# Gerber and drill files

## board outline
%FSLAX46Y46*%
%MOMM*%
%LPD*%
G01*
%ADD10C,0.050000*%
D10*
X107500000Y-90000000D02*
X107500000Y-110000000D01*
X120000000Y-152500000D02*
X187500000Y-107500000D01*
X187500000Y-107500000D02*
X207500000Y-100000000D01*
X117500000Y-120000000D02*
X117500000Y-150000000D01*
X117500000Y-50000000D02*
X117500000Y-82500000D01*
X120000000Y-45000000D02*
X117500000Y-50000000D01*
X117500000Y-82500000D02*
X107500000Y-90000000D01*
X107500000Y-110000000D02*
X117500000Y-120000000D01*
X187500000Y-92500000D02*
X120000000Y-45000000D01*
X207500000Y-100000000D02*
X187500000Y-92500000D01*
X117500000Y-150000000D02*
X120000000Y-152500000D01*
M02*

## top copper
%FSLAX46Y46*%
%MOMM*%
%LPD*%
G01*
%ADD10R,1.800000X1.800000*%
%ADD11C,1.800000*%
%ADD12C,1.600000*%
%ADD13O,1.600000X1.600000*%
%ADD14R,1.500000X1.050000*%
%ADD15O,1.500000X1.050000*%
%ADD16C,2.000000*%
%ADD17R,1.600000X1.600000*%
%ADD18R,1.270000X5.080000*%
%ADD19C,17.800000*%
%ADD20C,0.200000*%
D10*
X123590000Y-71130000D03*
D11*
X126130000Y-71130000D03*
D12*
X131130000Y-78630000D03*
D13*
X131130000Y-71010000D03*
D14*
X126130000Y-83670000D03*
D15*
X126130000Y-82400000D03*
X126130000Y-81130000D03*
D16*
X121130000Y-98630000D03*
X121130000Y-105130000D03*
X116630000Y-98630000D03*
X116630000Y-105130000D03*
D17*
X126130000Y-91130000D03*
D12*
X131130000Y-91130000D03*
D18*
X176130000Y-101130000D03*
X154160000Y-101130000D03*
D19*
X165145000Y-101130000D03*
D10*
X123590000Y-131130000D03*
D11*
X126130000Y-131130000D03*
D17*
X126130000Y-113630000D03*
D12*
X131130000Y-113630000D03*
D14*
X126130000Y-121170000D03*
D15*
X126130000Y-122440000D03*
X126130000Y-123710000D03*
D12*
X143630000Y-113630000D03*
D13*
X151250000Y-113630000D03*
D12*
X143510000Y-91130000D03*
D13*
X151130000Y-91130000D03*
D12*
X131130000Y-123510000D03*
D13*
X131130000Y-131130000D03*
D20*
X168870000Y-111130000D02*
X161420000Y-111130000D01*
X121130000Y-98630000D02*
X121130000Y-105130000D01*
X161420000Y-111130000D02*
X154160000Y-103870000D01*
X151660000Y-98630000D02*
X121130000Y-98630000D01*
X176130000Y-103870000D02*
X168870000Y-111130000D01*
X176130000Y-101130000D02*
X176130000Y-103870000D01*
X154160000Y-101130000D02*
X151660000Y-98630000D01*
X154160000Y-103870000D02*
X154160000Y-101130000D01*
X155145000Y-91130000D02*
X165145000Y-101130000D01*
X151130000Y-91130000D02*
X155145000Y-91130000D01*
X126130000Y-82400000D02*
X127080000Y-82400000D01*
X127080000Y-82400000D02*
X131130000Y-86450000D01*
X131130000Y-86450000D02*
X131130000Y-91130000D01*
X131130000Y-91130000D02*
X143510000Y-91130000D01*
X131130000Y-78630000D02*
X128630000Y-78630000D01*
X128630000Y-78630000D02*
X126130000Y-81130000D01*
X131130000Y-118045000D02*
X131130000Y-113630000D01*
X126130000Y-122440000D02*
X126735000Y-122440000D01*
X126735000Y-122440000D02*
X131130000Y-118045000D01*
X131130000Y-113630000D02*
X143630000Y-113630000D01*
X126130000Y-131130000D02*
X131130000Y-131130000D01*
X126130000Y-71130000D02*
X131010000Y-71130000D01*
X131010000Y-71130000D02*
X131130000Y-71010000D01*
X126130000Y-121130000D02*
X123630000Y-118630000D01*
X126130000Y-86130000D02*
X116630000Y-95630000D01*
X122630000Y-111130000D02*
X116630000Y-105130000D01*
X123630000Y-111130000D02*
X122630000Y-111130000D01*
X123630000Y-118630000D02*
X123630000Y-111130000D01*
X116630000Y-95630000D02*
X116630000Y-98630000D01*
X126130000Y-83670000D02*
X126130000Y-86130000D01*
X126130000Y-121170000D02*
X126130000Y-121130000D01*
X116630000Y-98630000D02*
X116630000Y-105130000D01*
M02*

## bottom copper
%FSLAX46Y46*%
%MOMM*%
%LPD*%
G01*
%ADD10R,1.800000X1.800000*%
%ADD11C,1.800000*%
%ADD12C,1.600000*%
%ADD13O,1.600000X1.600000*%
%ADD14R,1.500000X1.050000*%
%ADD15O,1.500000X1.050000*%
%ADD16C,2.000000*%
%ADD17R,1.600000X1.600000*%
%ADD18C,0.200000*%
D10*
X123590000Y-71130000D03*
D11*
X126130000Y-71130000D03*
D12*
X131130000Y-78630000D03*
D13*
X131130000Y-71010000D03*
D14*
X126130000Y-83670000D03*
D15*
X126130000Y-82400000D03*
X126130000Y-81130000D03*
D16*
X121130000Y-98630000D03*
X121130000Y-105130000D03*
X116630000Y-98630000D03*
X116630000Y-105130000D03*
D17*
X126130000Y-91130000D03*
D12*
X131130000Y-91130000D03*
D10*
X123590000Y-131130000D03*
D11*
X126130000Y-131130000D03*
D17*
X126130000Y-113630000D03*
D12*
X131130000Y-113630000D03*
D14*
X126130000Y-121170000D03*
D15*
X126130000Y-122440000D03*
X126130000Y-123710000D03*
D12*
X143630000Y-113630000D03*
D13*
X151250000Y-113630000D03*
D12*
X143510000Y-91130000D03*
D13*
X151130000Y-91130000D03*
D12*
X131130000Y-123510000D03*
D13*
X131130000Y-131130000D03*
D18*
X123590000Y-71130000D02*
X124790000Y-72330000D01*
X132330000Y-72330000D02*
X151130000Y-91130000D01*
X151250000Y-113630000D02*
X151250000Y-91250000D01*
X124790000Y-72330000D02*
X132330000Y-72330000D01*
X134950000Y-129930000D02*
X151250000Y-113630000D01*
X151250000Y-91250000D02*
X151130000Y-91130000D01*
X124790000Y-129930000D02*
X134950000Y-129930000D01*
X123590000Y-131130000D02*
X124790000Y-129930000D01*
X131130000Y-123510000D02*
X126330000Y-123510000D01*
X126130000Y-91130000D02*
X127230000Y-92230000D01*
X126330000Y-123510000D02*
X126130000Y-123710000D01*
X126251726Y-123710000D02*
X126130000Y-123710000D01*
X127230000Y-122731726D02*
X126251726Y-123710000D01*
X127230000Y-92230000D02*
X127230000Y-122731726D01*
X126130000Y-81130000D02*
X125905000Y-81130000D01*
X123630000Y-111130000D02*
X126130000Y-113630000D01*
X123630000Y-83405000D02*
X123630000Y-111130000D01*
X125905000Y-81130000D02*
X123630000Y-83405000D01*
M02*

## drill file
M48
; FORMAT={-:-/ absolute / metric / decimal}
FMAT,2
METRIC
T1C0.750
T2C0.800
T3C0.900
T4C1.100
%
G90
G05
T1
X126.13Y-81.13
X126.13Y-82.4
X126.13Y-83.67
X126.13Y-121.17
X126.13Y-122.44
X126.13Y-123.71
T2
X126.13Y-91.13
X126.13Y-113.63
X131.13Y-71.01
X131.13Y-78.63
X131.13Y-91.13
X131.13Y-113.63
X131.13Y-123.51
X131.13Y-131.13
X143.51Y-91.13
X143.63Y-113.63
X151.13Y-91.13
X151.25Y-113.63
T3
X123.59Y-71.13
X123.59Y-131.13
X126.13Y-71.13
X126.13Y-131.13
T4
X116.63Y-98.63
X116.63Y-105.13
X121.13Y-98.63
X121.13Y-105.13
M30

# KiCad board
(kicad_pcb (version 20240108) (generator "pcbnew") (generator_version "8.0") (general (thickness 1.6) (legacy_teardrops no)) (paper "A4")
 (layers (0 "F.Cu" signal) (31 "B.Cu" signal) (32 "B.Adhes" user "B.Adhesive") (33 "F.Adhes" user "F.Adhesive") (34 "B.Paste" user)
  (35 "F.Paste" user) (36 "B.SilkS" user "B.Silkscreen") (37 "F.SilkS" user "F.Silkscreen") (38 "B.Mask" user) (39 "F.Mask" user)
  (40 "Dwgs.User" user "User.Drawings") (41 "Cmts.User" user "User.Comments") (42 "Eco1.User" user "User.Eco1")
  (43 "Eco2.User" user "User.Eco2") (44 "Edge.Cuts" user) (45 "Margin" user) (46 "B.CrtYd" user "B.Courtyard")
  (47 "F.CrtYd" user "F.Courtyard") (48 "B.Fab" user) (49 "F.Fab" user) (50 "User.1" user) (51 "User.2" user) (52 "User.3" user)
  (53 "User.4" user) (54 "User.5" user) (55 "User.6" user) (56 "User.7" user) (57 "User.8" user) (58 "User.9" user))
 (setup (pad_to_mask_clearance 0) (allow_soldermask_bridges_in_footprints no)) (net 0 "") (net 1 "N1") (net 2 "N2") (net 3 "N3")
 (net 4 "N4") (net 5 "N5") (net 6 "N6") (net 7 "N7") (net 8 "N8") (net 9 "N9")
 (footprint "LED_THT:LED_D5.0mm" (layer "F.Cu") (at 123.59 71.13)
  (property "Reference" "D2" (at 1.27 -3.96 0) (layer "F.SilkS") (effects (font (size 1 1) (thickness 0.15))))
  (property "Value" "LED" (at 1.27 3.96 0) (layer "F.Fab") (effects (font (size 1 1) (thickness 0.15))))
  (pad "1" thru_hole rect (at 0 0) (size 1.8 1.8) (drill 0.9) (layers "*.Cu" "*.Mask") (remove_unused_layers no) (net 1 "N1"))
  (pad "2" thru_hole circle (at 2.54 0) (size 1.8 1.8) (drill 0.9) (layers "*.Cu" "*.Mask") (remove_unused_layers no) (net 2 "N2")))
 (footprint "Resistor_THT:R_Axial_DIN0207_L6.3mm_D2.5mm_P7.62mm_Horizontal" (layer "F.Cu") (at 131.13 78.63 90)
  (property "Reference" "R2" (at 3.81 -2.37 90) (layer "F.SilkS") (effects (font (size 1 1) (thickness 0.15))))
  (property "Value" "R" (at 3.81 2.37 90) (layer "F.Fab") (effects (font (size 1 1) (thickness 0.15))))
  (pad "1" thru_hole circle (at 0 0 90) (size 1.6 1.6) (drill 0.8) (layers "*.Cu" "*.Mask") (remove_unused_layers no) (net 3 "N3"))
  (pad "2" thru_hole oval (at 7.62 0 90) (size 1.6 1.6) (drill 0.8) (layers "*.Cu" "*.Mask") (remove_unused_layers no) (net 2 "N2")))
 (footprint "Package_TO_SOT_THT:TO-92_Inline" (layer "F.Cu") (at 126.13 83.67 90)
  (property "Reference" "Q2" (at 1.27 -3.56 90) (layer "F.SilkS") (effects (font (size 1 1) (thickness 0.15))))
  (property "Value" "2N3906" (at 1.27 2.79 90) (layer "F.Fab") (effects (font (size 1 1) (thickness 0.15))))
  (pad "1" thru_hole rect (at 0 0 90) (size 1.05 1.5) (drill 0.75) (layers "*.Cu" "*.Mask") (remove_unused_layers no) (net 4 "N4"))
  (pad "2" thru_hole oval (at 1.27 0 90) (size 1.05 1.5) (drill 0.75) (layers "*.Cu" "*.Mask") (remove_unused_layers no) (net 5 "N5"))
  (pad "3" thru_hole oval (at 2.54 0 90) (size 1.05 1.5) (drill 0.75) (layers "*.Cu" "*.Mask") (remove_unused_layers no) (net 3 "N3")))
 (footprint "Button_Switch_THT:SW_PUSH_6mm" (layer "F.Cu") (at 121.13 98.63 -90)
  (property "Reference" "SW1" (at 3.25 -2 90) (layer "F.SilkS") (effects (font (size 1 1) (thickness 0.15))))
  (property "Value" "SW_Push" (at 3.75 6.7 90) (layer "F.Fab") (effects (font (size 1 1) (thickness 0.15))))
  (pad "1" thru_hole circle (at 0 0) (size 2 2) (drill 1.1) (layers "*.Cu" "*.Mask") (remove_unused_layers no) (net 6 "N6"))
  (pad "1" thru_hole circle (at 6.5 0) (size 2 2) (drill 1.1) (layers "*.Cu" "*.Mask") (remove_unused_layers no) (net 6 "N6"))
  (pad "2" thru_hole circle (at 0 4.5) (size 2 2) (drill 1.1) (layers "*.Cu" "*.Mask") (remove_unused_layers no) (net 4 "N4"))
  (pad "2" thru_hole circle (at 6.5 4.5) (size 2 2) (drill 1.1) (layers "*.Cu" "*.Mask") (remove_unused_layers no) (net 4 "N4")))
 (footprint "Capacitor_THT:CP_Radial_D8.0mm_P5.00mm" (layer "F.Cu") (at 126.13 91.13)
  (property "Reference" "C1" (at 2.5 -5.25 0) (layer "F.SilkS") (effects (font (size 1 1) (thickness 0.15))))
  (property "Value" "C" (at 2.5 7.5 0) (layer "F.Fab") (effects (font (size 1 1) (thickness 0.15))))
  (pad "1" thru_hole rect (at 0 0) (size 1.6 1.6) (drill 0.8) (layers "*.Cu" "*.Mask") (remove_unused_layers no) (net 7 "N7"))
  (pad "2" thru_hole circle (at 5 0) (size 1.6 1.6) (drill 0.8) (layers "*.Cu" "*.Mask") (remove_unused_layers no) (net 5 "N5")))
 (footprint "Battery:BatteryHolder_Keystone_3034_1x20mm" (layer "F.Cu") (at 165.145 101.13 180)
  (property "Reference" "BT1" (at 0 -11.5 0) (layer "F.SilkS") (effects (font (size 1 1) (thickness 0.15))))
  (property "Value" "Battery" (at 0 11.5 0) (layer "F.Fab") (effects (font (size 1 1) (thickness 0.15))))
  (pad "1" smd rect (at -10.985 0 180) (size 1.27 5.08) (layers "F.Cu" "F.Paste" "F.Mask") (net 6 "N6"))
  (pad "1" smd rect (at 10.985 0 180) (size 1.27 5.08) (layers "F.Cu" "F.Paste" "F.Mask") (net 6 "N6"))
  (pad "2" smd circle (at 0 0 180) (size 17.8 17.8) (layers "F.Cu" "F.Mask") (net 1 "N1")))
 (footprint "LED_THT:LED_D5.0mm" (layer "F.Cu") (at 123.59 131.13)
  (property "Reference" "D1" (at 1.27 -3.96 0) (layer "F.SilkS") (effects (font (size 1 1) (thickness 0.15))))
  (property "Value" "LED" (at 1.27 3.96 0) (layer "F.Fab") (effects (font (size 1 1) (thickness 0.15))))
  (pad "1" thru_hole rect (at 0 0) (size 1.8 1.8) (drill 0.9) (layers "*.Cu" "*.Mask") (remove_unused_layers no) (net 1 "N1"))
  (pad "2" thru_hole circle (at 2.54 0) (size 1.8 1.8) (drill 0.9) (layers "*.Cu" "*.Mask") (remove_unused_layers no) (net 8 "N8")))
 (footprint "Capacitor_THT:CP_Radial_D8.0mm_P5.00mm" (layer "F.Cu") (at 126.13 113.63)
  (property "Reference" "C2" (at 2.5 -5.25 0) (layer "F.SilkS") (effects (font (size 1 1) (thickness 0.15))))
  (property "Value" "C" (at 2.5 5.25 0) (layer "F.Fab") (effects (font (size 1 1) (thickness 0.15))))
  (pad "1" thru_hole rect (at 0 0) (size 1.6 1.6) (drill 0.8) (layers "*.Cu" "*.Mask") (remove_unused_layers no) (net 3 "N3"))
  (pad "2" thru_hole circle (at 5 0) (size 1.6 1.6) (drill 0.8) (layers "*.Cu" "*.Mask") (remove_unused_layers no) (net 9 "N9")))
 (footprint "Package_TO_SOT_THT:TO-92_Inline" (layer "F.Cu") (at 126.13 121.17 -90)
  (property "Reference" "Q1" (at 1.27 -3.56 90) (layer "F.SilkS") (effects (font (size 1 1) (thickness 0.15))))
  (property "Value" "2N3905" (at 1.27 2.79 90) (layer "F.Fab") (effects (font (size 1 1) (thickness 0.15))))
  (pad "1" thru_hole rect (at 0 0 270) (size 1.05 1.5) (drill 0.75) (layers "*.Cu" "*.Mask") (remove_unused_layers no) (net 4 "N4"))
  (pad "2" thru_hole oval (at 1.27 0 270) (size 1.05 1.5) (drill 0.75) (layers "*.Cu" "*.Mask") (remove_unused_layers no) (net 9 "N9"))
  (pad "3" thru_hole oval (at 2.54 0 270) (size 1.05 1.5) (drill 0.75) (layers "*.Cu" "*.Mask") (remove_unused_layers no) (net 7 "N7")))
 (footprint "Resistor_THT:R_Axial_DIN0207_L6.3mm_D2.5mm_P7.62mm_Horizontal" (layer "F.Cu") (at 143.63 113.63)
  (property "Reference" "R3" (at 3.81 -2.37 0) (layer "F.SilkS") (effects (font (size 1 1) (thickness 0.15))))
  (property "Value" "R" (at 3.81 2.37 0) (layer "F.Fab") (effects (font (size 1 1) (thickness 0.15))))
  (pad "1" thru_hole circle (at 0 0) (size 1.6 1.6) (drill 0.8) (layers "*.Cu" "*.Mask") (remove_unused_layers no) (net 9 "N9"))
  (pad "2" thru_hole oval (at 7.62 0) (size 1.6 1.6) (drill 0.8) (layers "*.Cu" "*.Mask") (remove_unused_layers no) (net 1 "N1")))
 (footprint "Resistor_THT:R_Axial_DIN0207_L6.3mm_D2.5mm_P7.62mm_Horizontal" (layer "F.Cu") (at 143.51 91.13)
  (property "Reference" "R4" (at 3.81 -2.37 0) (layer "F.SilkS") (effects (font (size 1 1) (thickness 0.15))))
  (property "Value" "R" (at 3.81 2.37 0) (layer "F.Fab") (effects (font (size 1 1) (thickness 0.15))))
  (pad "1" thru_hole circle (at 0 0) (size 1.6 1.6) (drill 0.8) (layers "*.Cu" "*.Mask") (remove_unused_layers no) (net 5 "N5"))
  (pad "2" thru_hole oval (at 7.62 0) (size 1.6 1.6) (drill 0.8) (layers "*.Cu" "*.Mask") (remove_unused_layers no) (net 1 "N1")))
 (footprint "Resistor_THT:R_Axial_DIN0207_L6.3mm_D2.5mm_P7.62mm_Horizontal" (layer "F.Cu") (at 131.13 123.51 -90)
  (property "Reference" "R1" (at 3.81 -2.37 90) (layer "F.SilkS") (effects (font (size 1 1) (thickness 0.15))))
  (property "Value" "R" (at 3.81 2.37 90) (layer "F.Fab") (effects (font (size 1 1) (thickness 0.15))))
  (pad "1" thru_hole circle (at 0 0 270) (size 1.6 1.6) (drill 0.8) (layers "*.Cu" "*.Mask") (remove_unused_layers no) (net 7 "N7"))
  (pad "2" thru_hole oval (at 7.62 0 270) (size 1.6 1.6) (drill 0.8) (layers "*.Cu" "*.Mask") (remove_unused_layers no) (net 8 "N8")))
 (gr_line (start 107.5 90) (end 107.5 110) (stroke (width 0.05) (type default)) (layer "Edge.Cuts"))
 (gr_line (start 120 152.5) (end 187.5 107.5) (stroke (width 0.05) (type default)) (layer "Edge.Cuts"))
 (gr_line (start 187.5 107.5) (end 207.5 100) (stroke (width 0.05) (type default)) (layer "Edge.Cuts"))
 (gr_line (start 117.5 120) (end 117.5 150) (stroke (width 0.05) (type default)) (layer "Edge.Cuts"))
 (gr_line (start 117.5 50) (end 117.5 82.5) (stroke (width 0.05) (type default)) (layer "Edge.Cuts"))
 (gr_line (start 120 45) (end 117.5 50) (stroke (width 0.05) (type default)) (layer "Edge.Cuts"))
 (gr_line (start 117.5 82.5) (end 107.5 90) (stroke (width 0.05) (type default)) (layer "Edge.Cuts"))
 (gr_line (start 107.5 110) (end 117.5 120) (stroke (width 0.05) (type default)) (layer "Edge.Cuts"))
 (gr_line (start 187.5 92.5) (end 120 45) (stroke (width 0.05) (type default)) (layer "Edge.Cuts"))
 (gr_line (start 207.5 100) (end 187.5 92.5) (stroke (width 0.05) (type default)) (layer "Edge.Cuts"))
 (gr_line (start 117.5 150) (end 120 152.5) (stroke (width 0.05) (type default)) (layer "Edge.Cuts"))
 (segment (start 168.87 111.13) (end 161.42 111.13) (width 0.2) (layer "F.Cu") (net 6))
 (segment (start 121.13 98.63) (end 121.13 105.13) (width 0.2) (layer "F.Cu") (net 6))
 (segment (start 161.42 111.13) (end 154.16 103.87) (width 0.2) (layer "F.Cu") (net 6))
 (segment (start 151.66 98.63) (end 121.13 98.63) (width 0.2) (layer "F.Cu") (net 6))
 (segment (start 176.13 103.87) (end 168.87 111.13) (width 0.2) (layer "F.Cu") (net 6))
 (segment (start 176.13 101.13) (end 176.13 103.87) (width 0.2) (layer "F.Cu") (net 6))
 (segment (start 154.16 101.13) (end 151.66 98.63) (width 0.2) (layer "F.Cu") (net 6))
 (segment (start 154.16 103.87) (end 154.16 101.13) (width 0.2) (layer "F.Cu") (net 6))
 (segment (start 155.145 91.13) (end 165.145 101.13) (width 0.2) (layer "F.Cu") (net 1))
 (segment (start 151.13 91.13) (end 155.145 91.13) (width 0.2) (layer "F.Cu") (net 1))
 (segment (start 123.59 71.13) (end 124.79 72.33) (width 0.2) (layer "B.Cu") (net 1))
 (segment (start 132.33 72.33) (end 151.13 91.13) (width 0.2) (layer "B.Cu") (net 1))
 (segment (start 151.25 113.63) (end 151.25 91.25) (width 0.2) (layer "B.Cu") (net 1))
 (segment (start 124.79 72.33) (end 132.33 72.33) (width 0.2) (layer "B.Cu") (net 1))
 (segment (start 134.95 129.93) (end 151.25 113.63) (width 0.2) (layer "B.Cu") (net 1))
 (segment (start 151.25 91.25) (end 151.13 91.13) (width 0.2) (layer "B.Cu") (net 1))
 (segment (start 124.79 129.93) (end 134.95 129.93) (width 0.2) (layer "B.Cu") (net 1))
 (segment (start 123.59 131.13) (end 124.79 129.93) (width 0.2) (layer "B.Cu") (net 1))
 (segment (start 126.13 82.4) (end 127.08 82.4) (width 0.2) (layer "F.Cu") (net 5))
 (segment (start 127.08 82.4) (end 131.13 86.45) (width 0.2) (layer "F.Cu") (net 5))
 (segment (start 131.13 86.45) (end 131.13 91.13) (width 0.2) (layer "F.Cu") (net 5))
 (segment (start 131.13 91.13) (end 143.51 91.13) (width 0.2) (layer "F.Cu") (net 5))
 (segment (start 131.13 123.51) (end 126.33 123.51) (width 0.2) (layer "B.Cu") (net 7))
 (segment (start 126.13 91.13) (end 127.23 92.23) (width 0.2) (layer "B.Cu") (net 7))
 (segment (start 126.33 123.51) (end 126.13 123.71) (width 0.2) (layer "B.Cu") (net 7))
 (segment (start 126.251726 123.71) (end 126.13 123.71) (width 0.2) (layer "B.Cu") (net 7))
 (segment (start 127.23 122.731726) (end 126.251726 123.71) (width 0.2) (layer "B.Cu") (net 7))
 (segment (start 127.23 92.23) (end 127.23 122.731726) (width 0.2) (layer "B.Cu") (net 7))
 (segment (start 131.13 78.63) (end 128.63 78.63) (width 0.2) (layer "F.Cu") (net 3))
 (segment (start 128.63 78.63) (end 126.13 81.13) (width 0.2) (layer "F.Cu") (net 3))
 (segment (start 126.13 81.13) (end 125.905 81.13) (width 0.2) (layer "B.Cu") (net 3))
 (segment (start 123.63 111.13) (end 126.13 113.63) (width 0.2) (layer "B.Cu") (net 3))
 (segment (start 123.63 83.405) (end 123.63 111.13) (width 0.2) (layer "B.Cu") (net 3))
 (segment (start 125.905 81.13) (end 123.63 83.405) (width 0.2) (layer "B.Cu") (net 3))
 (segment (start 131.13 118.045) (end 131.13 113.63) (width 0.2) (layer "F.Cu") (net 9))
 (segment (start 126.13 122.44) (end 126.735 122.44) (width 0.2) (layer "F.Cu") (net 9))
 (segment (start 126.735 122.44) (end 131.13 118.045) (width 0.2) (layer "F.Cu") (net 9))
 (segment (start 131.13 113.63) (end 143.63 113.63) (width 0.2) (layer "F.Cu") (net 9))
 (segment (start 126.13 131.13) (end 131.13 131.13) (width 0.2) (layer "F.Cu") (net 8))
 (segment (start 126.13 71.13) (end 131.01 71.13) (width 0.2) (layer "F.Cu") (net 2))
 (segment (start 131.01 71.13) (end 131.13 71.01) (width 0.2) (layer "F.Cu") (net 2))
 (segment (start 126.13 121.13) (end 123.63 118.63) (width 0.2) (layer "F.Cu") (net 4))
 (segment (start 126.13 86.13) (end 116.63 95.63) (width 0.2) (layer "F.Cu") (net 4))
 (segment (start 122.63 111.13) (end 116.63 105.13) (width 0.2) (layer "F.Cu") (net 4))
 (segment (start 123.63 111.13) (end 122.63 111.13) (width 0.2) (layer "F.Cu") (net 4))
 (segment (start 123.63 118.63) (end 123.63 111.13) (width 0.2) (layer "F.Cu") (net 4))
 (segment (start 116.63 95.63) (end 116.63 98.63) (width 0.2) (layer "F.Cu") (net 4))
 (segment (start 126.13 83.67) (end 126.13 86.13) (width 0.2) (layer "F.Cu") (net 4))
 (segment (start 126.13 121.17) (end 126.13 121.13) (width 0.2) (layer "F.Cu") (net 4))
 (segment (start 116.63 98.63) (end 116.63 105.13) (width 0.2) (layer "F.Cu") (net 4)))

